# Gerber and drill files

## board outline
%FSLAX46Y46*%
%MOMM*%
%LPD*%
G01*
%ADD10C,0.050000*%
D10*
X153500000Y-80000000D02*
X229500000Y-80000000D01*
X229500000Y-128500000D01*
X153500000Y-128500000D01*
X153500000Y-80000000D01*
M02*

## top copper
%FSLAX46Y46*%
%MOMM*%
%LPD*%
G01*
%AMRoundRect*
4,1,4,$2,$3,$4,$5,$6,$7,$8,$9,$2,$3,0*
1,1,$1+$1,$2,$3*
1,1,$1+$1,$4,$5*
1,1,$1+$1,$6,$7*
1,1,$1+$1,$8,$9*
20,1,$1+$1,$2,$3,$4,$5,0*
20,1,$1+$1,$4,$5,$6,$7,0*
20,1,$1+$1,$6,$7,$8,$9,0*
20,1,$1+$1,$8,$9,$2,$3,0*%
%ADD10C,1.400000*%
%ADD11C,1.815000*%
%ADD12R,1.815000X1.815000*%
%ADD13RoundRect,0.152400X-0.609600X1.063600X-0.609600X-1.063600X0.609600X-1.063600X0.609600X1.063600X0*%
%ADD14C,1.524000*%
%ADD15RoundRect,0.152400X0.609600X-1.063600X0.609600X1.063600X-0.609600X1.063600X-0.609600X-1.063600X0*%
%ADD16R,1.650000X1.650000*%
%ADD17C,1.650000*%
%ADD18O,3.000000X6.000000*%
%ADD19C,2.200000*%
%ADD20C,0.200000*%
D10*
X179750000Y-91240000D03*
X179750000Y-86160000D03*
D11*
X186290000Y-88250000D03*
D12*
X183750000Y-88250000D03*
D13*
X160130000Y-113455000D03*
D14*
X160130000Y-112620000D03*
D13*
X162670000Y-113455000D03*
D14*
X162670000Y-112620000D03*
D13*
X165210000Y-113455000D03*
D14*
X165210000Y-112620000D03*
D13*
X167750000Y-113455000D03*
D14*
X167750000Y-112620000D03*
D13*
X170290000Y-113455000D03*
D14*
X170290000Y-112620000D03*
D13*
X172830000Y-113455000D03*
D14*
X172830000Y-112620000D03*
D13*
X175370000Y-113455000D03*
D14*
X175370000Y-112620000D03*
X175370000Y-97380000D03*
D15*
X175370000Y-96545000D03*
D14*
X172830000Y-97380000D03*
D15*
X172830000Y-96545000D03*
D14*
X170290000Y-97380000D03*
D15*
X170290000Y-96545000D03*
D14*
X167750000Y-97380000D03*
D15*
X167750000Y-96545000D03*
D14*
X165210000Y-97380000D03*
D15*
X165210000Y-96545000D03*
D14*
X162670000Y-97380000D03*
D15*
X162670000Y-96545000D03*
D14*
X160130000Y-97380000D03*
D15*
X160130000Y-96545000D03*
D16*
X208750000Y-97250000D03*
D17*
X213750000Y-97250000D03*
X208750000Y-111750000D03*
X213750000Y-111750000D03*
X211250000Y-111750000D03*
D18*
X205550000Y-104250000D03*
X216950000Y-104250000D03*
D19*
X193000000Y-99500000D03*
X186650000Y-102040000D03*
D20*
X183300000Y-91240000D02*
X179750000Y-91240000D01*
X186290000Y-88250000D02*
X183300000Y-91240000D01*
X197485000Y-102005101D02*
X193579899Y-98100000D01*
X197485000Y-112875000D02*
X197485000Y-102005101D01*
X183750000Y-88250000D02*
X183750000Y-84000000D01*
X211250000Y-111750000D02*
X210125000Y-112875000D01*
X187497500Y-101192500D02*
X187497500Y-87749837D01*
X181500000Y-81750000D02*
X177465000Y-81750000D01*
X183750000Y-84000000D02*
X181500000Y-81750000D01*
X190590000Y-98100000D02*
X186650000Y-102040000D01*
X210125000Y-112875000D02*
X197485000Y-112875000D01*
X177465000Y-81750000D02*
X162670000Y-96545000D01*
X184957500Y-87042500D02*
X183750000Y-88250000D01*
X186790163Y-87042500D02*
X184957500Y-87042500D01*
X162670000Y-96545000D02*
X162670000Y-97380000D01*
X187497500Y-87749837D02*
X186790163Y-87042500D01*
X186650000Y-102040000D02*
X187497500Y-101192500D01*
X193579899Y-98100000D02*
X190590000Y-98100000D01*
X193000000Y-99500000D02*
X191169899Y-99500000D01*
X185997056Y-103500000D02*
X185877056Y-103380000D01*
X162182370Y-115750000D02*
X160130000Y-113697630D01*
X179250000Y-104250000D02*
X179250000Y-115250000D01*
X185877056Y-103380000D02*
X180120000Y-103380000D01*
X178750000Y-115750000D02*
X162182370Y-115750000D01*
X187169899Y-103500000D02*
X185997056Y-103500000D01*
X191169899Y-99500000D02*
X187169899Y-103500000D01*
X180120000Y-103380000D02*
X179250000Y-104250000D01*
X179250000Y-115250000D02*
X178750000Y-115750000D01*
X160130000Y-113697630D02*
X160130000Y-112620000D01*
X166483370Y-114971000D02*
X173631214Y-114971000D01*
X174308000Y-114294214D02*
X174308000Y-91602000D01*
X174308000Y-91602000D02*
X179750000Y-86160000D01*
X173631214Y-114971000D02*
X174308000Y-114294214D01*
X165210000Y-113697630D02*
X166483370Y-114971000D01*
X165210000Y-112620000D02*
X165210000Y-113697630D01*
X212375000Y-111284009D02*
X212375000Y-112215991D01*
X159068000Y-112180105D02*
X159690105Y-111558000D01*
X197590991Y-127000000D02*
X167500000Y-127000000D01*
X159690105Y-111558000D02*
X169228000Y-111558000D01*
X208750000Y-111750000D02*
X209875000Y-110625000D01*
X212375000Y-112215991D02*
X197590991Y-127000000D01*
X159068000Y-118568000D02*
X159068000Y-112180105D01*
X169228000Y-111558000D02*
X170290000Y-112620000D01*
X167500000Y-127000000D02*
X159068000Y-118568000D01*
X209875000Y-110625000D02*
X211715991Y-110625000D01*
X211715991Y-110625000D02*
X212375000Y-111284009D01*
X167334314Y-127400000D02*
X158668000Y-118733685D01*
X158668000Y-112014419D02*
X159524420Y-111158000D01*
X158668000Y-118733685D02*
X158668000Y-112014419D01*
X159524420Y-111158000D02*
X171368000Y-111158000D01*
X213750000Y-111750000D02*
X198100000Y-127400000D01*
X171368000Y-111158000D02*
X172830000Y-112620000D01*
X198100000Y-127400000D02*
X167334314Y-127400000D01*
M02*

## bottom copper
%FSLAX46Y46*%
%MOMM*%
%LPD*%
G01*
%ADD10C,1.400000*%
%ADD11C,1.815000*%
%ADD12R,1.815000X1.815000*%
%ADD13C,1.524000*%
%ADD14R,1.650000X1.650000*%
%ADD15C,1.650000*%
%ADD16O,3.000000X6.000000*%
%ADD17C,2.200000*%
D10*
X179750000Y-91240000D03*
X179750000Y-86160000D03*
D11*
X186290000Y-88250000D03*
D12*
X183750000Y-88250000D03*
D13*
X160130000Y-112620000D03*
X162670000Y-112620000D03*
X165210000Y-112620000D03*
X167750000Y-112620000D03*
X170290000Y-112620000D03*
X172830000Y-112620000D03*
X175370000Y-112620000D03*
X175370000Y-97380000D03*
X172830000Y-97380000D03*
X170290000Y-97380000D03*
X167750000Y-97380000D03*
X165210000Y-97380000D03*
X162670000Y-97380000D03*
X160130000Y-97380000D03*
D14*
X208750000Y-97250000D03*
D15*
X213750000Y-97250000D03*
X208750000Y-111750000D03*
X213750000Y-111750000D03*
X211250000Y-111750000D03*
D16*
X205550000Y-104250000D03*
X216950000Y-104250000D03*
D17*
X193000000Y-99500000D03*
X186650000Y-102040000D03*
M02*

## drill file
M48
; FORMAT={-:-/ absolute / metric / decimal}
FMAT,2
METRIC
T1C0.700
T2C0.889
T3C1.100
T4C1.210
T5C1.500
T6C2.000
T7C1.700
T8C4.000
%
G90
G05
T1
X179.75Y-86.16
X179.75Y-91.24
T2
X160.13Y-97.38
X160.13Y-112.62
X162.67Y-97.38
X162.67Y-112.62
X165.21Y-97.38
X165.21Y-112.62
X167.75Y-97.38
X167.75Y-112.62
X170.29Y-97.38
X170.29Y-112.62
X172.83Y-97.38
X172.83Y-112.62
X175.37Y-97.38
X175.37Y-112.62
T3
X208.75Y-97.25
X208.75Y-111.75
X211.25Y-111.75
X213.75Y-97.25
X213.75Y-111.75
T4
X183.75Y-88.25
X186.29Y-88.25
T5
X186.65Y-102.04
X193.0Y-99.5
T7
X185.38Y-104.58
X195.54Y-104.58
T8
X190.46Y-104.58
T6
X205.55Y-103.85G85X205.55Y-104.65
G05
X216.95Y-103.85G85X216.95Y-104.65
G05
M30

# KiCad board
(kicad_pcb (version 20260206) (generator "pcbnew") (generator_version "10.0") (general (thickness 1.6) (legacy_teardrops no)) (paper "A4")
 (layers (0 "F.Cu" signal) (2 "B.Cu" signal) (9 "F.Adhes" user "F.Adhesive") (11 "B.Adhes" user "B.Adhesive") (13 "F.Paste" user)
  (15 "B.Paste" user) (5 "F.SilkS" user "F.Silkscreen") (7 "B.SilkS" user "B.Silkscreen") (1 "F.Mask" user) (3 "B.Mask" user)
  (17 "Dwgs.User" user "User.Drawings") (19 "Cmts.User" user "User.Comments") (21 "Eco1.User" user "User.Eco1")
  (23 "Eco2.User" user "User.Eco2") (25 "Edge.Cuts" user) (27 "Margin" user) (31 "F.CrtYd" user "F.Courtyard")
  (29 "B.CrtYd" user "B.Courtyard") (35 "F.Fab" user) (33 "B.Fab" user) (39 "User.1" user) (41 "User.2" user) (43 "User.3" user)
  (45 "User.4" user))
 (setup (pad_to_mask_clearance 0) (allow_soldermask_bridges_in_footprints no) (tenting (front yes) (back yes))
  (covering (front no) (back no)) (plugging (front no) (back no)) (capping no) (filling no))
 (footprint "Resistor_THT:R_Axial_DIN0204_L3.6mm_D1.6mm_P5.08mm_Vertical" (layer "F.Cu") (at 179.75 91.24 90)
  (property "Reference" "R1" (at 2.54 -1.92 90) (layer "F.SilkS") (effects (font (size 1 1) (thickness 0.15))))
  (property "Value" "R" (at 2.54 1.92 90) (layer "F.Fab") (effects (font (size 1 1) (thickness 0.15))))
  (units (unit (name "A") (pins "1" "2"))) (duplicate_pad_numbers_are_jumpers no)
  (pad "1" thru_hole circle (at 0 0 90) (size 1.4 1.4) (drill 0.7) (layers "*.Cu" "*.Mask") (remove_unused_layers no) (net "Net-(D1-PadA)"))
  (pad "2" thru_hole circle (at 5.08 0 90) (size 1.4 1.4) (drill 0.7) (layers "*.Cu" "*.Mask") (remove_unused_layers no) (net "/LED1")))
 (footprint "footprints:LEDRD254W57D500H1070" (layer "F.Cu") (at 185.02 88.25)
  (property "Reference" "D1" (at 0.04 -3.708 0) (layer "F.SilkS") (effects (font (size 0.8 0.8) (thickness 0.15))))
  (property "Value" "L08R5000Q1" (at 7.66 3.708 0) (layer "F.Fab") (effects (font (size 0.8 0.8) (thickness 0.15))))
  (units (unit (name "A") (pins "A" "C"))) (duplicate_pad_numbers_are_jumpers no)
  (pad "A" thru_hole circle (at 1.27 0) (size 1.815 1.815) (drill 1.21) (layers "*.Cu" "*.Mask") (remove_unused_layers no)
   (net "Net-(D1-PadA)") (solder_mask_margin 0.102))
  (pad "C" thru_hole rect (at -1.27 0) (size 1.815 1.815) (drill 1.21) (layers "*.Cu" "*.Mask") (remove_unused_layers no) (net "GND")
   (solder_mask_margin 0.102)))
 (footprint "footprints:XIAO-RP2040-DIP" (layer "F.Cu") (at 167.75 105 180)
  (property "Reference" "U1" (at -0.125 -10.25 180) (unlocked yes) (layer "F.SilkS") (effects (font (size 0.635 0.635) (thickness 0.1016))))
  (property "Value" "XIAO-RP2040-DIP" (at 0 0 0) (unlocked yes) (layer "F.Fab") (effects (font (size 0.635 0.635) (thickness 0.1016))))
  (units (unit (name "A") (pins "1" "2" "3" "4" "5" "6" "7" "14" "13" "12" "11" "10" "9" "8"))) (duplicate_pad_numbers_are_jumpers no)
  (pad "1" smd roundrect (at 7.62 -8.455 270) (size 2.432 1.524) (layers "F.Cu" "F.Mask") (roundrect_rratio 0.1) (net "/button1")
   (thermal_bridge_angle 45))
  (pad "1" thru_hole circle (at 7.62 -7.62 270) (size 1.524 1.524) (drill 0.889) (layers "*.Cu" "*.Mask") (remove_unused_layers no)
   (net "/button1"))
  (pad "2" smd roundrect (at 5.08 -8.455 270) (size 2.432 1.524) (layers "F.Cu" "F.Mask") (roundrect_rratio 0.1)
   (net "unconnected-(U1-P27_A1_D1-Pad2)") (thermal_bridge_angle 45))
  (pad "2" thru_hole circle (at 5.08 -7.62 270) (size 1.524 1.524) (drill 0.889) (layers "*.Cu" "*.Mask") (remove_unused_layers no)
   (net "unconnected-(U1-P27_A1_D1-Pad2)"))
  (pad "3" smd roundrect (at 2.54 -8.455 270) (size 2.432 1.524) (layers "F.Cu" "F.Mask") (roundrect_rratio 0.1) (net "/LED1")
   (thermal_bridge_angle 45))
  (pad "3" thru_hole circle (at 2.54 -7.62 270) (size 1.524 1.524) (drill 0.889) (layers "*.Cu" "*.Mask") (remove_unused_layers no)
   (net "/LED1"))
  (pad "4" smd roundrect (at 0 -8.455 270) (size 2.432 1.524) (layers "F.Cu" "F.Mask") (roundrect_rratio 0.1) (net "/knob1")
   (thermal_bridge_angle 45))
  (pad "4" thru_hole circle (at 0 -7.62 270) (size 1.524 1.524) (drill 0.889) (layers "*.Cu" "*.Mask") (remove_unused_layers no)
   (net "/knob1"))
  (pad "5" smd roundrect (at -2.54 -8.455 270) (size 2.432 1.524) (layers "F.Cu" "F.Mask") (roundrect_rratio 0.1) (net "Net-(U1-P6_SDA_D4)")
   (thermal_bridge_angle 45))
  (pad "5" thru_hole circle (at -2.54 -7.62 270) (size 1.524 1.524) (drill 0.889) (layers "*.Cu" "*.Mask") (remove_unused_layers no)
   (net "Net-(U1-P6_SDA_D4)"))
  (pad "6" smd roundrect (at -5.08 -8.455 270) (size 2.432 1.524) (layers "F.Cu" "F.Mask") (roundrect_rratio 0.1) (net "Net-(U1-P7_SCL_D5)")
   (thermal_bridge_angle 45))
  (pad "6" thru_hole circle (at -5.08 -7.62 270) (size 1.524 1.524) (drill 0.889) (layers "*.Cu" "*.Mask") (remove_unused_layers no)
   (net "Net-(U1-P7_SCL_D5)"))
  (pad "7" smd roundrect (at -7.62 -8.455 270) (size 2.432 1.524) (layers "F.Cu" "F.Mask") (roundrect_rratio 0.1)
   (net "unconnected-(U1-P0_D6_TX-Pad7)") (thermal_bridge_angle 45))
  (pad "7" thru_hole circle (at -7.62 -7.62 270) (size 1.524 1.524) (drill 0.889) (layers "*.Cu" "*.Mask") (remove_unused_layers no)
   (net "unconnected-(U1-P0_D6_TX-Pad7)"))
  (pad "8" thru_hole circle (at -7.62 7.62 90) (size 1.524 1.524) (drill 0.889) (layers "*.Cu" "*.Mask") (remove_unused_layers no)
   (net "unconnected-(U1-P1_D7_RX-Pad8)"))
  (pad "8" smd roundrect (at -7.62 8.455 90) (size 2.432 1.524) (layers "F.Cu" "F.Mask") (roundrect_rratio 0.1)
   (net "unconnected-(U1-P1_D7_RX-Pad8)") (thermal_bridge_angle 45))
  (pad "9" thru_hole circle (at -5.08 7.62 90) (size 1.524 1.524) (drill 0.889) (layers "*.Cu" "*.Mask") (remove_unused_layers no)
   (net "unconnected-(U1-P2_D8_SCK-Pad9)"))
  (pad "9" smd roundrect (at -5.08 8.455 90) (size 2.432 1.524) (layers "F.Cu" "F.Mask") (roundrect_rratio 0.1)
   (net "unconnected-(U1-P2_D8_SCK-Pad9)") (thermal_bridge_angle 45))
  (pad "10" thru_hole circle (at -2.54 7.62 90) (size 1.524 1.524) (drill 0.889) (layers "*.Cu" "*.Mask") (remove_unused_layers no)
   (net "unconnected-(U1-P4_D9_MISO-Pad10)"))
  (pad "10" smd roundrect (at -2.54 8.455 90) (size 2.432 1.524) (layers "F.Cu" "F.Mask") (roundrect_rratio 0.1)
   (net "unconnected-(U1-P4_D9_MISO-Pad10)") (thermal_bridge_angle 45))
  (pad "11" thru_hole circle (at 0 7.62 90) (size 1.524 1.524) (drill 0.889) (layers "*.Cu" "*.Mask") (remove_unused_layers no)
   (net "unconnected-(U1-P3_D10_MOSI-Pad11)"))
  (pad "11" smd roundrect (at 0 8.455 90) (size 2.432 1.524) (layers "F.Cu" "F.Mask") (roundrect_rratio 0.1)
   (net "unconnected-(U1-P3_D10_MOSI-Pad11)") (thermal_bridge_angle 45))
  (pad "12" thru_hole circle (at 2.54 7.62 90) (size 1.524 1.524) (drill 0.889) (layers "*.Cu" "*.Mask") (remove_unused_layers no)
   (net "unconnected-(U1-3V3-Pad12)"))
  (pad "12" smd roundrect (at 2.54 8.455 90) (size 2.432 1.524) (layers "F.Cu" "F.Mask") (roundrect_rratio 0.1)
   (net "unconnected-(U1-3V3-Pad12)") (thermal_bridge_angle 45))
  (pad "13" thru_hole circle (at 5.08 7.62 90) (size 1.524 1.524) (drill 0.889) (layers "*.Cu" "*.Mask") (remove_unused_layers no)
   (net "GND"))
  (pad "13" smd roundrect (at 5.08 8.455 90) (size 2.432 1.524) (layers "F.Cu" "F.Mask") (roundrect_rratio 0.1) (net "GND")
   (thermal_bridge_angle 45))
  (pad "14" thru_hole circle (at 7.62 7.62 90) (size 1.524 1.524) (drill 0.889) (layers "*.Cu" "*.Mask") (remove_unused_layers no)
   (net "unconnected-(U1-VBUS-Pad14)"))
  (pad "14" smd roundrect (at 7.62 8.455 90) (size 2.432 1.524) (layers "F.Cu" "F.Mask") (roundrect_rratio 0.1)
   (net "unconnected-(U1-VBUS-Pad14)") (thermal_bridge_angle 45)))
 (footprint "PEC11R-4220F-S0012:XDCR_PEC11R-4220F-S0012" (layer "F.Cu") (at 211.25 104.25)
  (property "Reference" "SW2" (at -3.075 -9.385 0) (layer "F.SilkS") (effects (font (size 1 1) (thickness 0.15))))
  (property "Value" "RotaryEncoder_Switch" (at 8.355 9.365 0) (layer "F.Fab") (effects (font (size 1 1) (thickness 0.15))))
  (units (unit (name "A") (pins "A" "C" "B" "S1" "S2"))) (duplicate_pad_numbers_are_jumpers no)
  (pad "1" thru_hole rect (at -2.5 -7) (size 1.65 1.65) (drill 1.1) (layers "*.Cu" "*.Mask") (remove_unused_layers no)
   (solder_mask_margin 0.102))
  (pad "2" thru_hole circle (at 2.5 -7) (size 1.65 1.65) (drill 1.1) (layers "*.Cu" "*.Mask") (remove_unused_layers no)
   (solder_mask_margin 0.102))
  (pad "A" thru_hole circle (at -2.5 7.5) (size 1.65 1.65) (drill 1.1) (layers "*.Cu" "*.Mask") (remove_unused_layers no)
   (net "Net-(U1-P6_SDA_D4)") (solder_mask_margin 0.102))
  (pad "B" thru_hole circle (at 2.5 7.5) (size 1.65 1.65) (drill 1.1) (layers "*.Cu" "*.Mask") (remove_unused_layers no)
   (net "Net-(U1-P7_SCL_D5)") (solder_mask_margin 0.102))
  (pad "C" thru_hole circle (at 0 7.5) (size 1.65 1.65) (drill 1.1) (layers "*.Cu" "*.Mask") (remove_unused_layers no) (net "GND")
   (solder_mask_margin 0.102))
  (pad "SH1" thru_hole oval (at -5.7 0) (size 3 6) (drill oval 2 2.8) (layers "*.Cu" "*.Mask") (remove_unused_layers no)
   (solder_mask_margin 0.102))
  (pad "SH2" thru_hole oval (at 5.7 0) (size 3 6) (drill oval 2 2.8) (layers "*.Cu" "*.Mask") (remove_unused_layers no)
   (solder_mask_margin 0.102)))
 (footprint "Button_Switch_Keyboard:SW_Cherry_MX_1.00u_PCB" (layer "F.Cu") (at 193 99.5)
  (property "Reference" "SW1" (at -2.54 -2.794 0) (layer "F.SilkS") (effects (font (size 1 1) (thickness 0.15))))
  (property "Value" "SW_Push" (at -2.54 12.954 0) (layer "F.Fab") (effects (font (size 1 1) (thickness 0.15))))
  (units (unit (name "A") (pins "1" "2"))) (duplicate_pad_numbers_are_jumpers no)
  (pad "" np_thru_hole circle (at -7.62 5.08) (size 1.7 1.7) (drill 1.7) (layers "*.Cu" "*.Mask"))
  (pad "" np_thru_hole circle (at -2.54 5.08) (size 4 4) (drill 4) (layers "*.Cu" "*.Mask"))
  (pad "" np_thru_hole circle (at 2.54 5.08) (size 1.7 1.7) (drill 1.7) (layers "*.Cu" "*.Mask"))
  (pad "1" thru_hole circle (at 0 0) (size 2.2 2.2) (drill 1.5) (layers "*.Cu" "*.Mask") (remove_unused_layers no) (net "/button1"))
  (pad "2" thru_hole circle (at -6.35 2.54) (size 2.2 2.2) (drill 1.5) (layers "*.Cu" "*.Mask") (remove_unused_layers no) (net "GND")))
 (gr_rect (start 153.5 80) (end 229.5 128.5) (stroke (width 0.05) (type default)) (fill no) (layer "Edge.Cuts"))
 (segment (start 183.3 91.24) (end 179.75 91.24) (width 0.2) (layer "F.Cu") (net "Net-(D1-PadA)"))
 (segment (start 186.29 88.25) (end 183.3 91.24) (width 0.2) (layer "F.Cu") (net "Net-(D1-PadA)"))
 (segment (start 197.485 102.005101) (end 193.579899 98.1) (width 0.2) (layer "F.Cu") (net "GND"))
 (segment (start 197.485 112.875) (end 197.485 102.005101) (width 0.2) (layer "F.Cu") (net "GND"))
 (segment (start 183.75 88.25) (end 183.75 84) (width 0.2) (layer "F.Cu") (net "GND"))
 (segment (start 211.25 111.75) (end 210.125 112.875) (width 0.2) (layer "F.Cu") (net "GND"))
 (segment (start 187.4975 101.1925) (end 187.4975 87.749837) (width 0.2) (layer "F.Cu") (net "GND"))
 (segment (start 181.5 81.75) (end 177.465 81.75) (width 0.2) (layer "F.Cu") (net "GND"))
 (segment (start 183.75 84) (end 181.5 81.75) (width 0.2) (layer "F.Cu") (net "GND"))
 (segment (start 190.59 98.1) (end 186.65 102.04) (width 0.2) (layer "F.Cu") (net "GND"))
 (segment (start 210.125 112.875) (end 197.485 112.875) (width 0.2) (layer "F.Cu") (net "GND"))
 (segment (start 177.465 81.75) (end 162.67 96.545) (width 0.2) (layer "F.Cu") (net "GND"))
 (segment (start 184.9575 87.0425) (end 183.75 88.25) (width 0.2) (layer "F.Cu") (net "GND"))
 (segment (start 186.790163 87.0425) (end 184.9575 87.0425) (width 0.2) (layer "F.Cu") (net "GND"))
 (segment (start 162.67 96.545) (end 162.67 97.38) (width 0.2) (layer "F.Cu") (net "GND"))
 (segment (start 187.4975 87.749837) (end 186.790163 87.0425) (width 0.2) (layer "F.Cu") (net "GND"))
 (segment (start 186.65 102.04) (end 187.4975 101.1925) (width 0.2) (layer "F.Cu") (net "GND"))
 (segment (start 193.579899 98.1) (end 190.59 98.1) (width 0.2) (layer "F.Cu") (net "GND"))
 (segment (start 193 99.5) (end 191.169899 99.5) (width 0.2) (layer "F.Cu") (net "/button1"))
 (segment (start 185.997056 103.5) (end 185.877056 103.38) (width 0.2) (layer "F.Cu") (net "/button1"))
 (segment (start 162.18237 115.75) (end 160.13 113.69763) (width 0.2) (layer "F.Cu") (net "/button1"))
 (segment (start 179.25 104.25) (end 179.25 115.25) (width 0.2) (layer "F.Cu") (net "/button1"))
 (segment (start 185.877056 103.38) (end 180.12 103.38) (width 0.2) (layer "F.Cu") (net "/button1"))
 (segment (start 178.75 115.75) (end 162.18237 115.75) (width 0.2) (layer "F.Cu") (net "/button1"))
 (segment (start 187.169899 103.5) (end 185.997056 103.5) (width 0.2) (layer "F.Cu") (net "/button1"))
 (segment (start 191.169899 99.5) (end 187.169899 103.5) (width 0.2) (layer "F.Cu") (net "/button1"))
 (segment (start 180.12 103.38) (end 179.25 104.25) (width 0.2) (layer "F.Cu") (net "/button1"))
 (segment (start 179.25 115.25) (end 178.75 115.75) (width 0.2) (layer "F.Cu") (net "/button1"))
 (segment (start 160.13 113.69763) (end 160.13 112.62) (width 0.2) (layer "F.Cu") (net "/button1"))
 (segment (start 166.48337 114.971) (end 173.631214 114.971) (width 0.2) (layer "F.Cu") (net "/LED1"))
 (segment (start 174.308 114.294214) (end 174.308 91.602) (width 0.2) (layer "F.Cu") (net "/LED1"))
 (segment (start 174.308 91.602) (end 179.75 86.16) (width 0.2) (layer "F.Cu") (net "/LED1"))
 (segment (start 173.631214 114.971) (end 174.308 114.294214) (width 0.2) (layer "F.Cu") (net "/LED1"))
 (segment (start 165.21 113.69763) (end 166.48337 114.971) (width 0.2) (layer "F.Cu") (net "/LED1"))
 (segment (start 165.21 112.62) (end 165.21 113.69763) (width 0.2) (layer "F.Cu") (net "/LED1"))
 (segment (start 212.375 111.284009) (end 212.375 112.215991) (width 0.2) (layer "F.Cu") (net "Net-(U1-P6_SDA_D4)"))
 (segment (start 159.068 112.180105) (end 159.690105 111.558) (width 0.2) (layer "F.Cu") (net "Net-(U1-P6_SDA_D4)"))
 (segment (start 197.590991 127) (end 167.5 127) (width 0.2) (layer "F.Cu") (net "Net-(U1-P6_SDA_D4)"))
 (segment (start 159.690105 111.558) (end 169.228 111.558) (width 0.2) (layer "F.Cu") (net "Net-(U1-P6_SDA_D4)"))
 (segment (start 208.75 111.75) (end 209.875 110.625) (width 0.2) (layer "F.Cu") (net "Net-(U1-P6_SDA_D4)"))
 (segment (start 212.375 112.215991) (end 197.590991 127) (width 0.2) (layer "F.Cu") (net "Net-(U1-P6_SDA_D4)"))
 (segment (start 159.068 118.568) (end 159.068 112.180105) (width 0.2) (layer "F.Cu") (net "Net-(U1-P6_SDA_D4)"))
 (segment (start 169.228 111.558) (end 170.29 112.62) (width 0.2) (layer "F.Cu") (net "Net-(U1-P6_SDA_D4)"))
 (segment (start 167.5 127) (end 159.068 118.568) (width 0.2) (layer "F.Cu") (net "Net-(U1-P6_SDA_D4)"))
 (segment (start 209.875 110.625) (end 211.715991 110.625) (width 0.2) (layer "F.Cu") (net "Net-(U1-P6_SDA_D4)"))
 (segment (start 211.715991 110.625) (end 212.375 111.284009) (width 0.2) (layer "F.Cu") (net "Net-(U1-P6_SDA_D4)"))
 (segment (start 167.334314 127.4) (end 158.668 118.733685) (width 0.2) (layer "F.Cu") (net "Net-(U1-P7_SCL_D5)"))
 (segment (start 158.668 112.014419) (end 159.52442 111.158) (width 0.2) (layer "F.Cu") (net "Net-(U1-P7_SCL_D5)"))
 (segment (start 158.668 118.733685) (end 158.668 112.014419) (width 0.2) (layer "F.Cu") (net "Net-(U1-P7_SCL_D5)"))
 (segment (start 159.52442 111.158) (end 171.368 111.158) (width 0.2) (layer "F.Cu") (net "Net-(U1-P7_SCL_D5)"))
 (segment (start 213.75 111.75) (end 198.1 127.4) (width 0.2) (layer "F.Cu") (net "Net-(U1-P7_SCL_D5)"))
 (segment (start 171.368 111.158) (end 172.83 112.62) (width 0.2) (layer "F.Cu") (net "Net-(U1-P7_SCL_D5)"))
 (segment (start 198.1 127.4) (end 167.334314 127.4) (width 0.2) (layer "F.Cu") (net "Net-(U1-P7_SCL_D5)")))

